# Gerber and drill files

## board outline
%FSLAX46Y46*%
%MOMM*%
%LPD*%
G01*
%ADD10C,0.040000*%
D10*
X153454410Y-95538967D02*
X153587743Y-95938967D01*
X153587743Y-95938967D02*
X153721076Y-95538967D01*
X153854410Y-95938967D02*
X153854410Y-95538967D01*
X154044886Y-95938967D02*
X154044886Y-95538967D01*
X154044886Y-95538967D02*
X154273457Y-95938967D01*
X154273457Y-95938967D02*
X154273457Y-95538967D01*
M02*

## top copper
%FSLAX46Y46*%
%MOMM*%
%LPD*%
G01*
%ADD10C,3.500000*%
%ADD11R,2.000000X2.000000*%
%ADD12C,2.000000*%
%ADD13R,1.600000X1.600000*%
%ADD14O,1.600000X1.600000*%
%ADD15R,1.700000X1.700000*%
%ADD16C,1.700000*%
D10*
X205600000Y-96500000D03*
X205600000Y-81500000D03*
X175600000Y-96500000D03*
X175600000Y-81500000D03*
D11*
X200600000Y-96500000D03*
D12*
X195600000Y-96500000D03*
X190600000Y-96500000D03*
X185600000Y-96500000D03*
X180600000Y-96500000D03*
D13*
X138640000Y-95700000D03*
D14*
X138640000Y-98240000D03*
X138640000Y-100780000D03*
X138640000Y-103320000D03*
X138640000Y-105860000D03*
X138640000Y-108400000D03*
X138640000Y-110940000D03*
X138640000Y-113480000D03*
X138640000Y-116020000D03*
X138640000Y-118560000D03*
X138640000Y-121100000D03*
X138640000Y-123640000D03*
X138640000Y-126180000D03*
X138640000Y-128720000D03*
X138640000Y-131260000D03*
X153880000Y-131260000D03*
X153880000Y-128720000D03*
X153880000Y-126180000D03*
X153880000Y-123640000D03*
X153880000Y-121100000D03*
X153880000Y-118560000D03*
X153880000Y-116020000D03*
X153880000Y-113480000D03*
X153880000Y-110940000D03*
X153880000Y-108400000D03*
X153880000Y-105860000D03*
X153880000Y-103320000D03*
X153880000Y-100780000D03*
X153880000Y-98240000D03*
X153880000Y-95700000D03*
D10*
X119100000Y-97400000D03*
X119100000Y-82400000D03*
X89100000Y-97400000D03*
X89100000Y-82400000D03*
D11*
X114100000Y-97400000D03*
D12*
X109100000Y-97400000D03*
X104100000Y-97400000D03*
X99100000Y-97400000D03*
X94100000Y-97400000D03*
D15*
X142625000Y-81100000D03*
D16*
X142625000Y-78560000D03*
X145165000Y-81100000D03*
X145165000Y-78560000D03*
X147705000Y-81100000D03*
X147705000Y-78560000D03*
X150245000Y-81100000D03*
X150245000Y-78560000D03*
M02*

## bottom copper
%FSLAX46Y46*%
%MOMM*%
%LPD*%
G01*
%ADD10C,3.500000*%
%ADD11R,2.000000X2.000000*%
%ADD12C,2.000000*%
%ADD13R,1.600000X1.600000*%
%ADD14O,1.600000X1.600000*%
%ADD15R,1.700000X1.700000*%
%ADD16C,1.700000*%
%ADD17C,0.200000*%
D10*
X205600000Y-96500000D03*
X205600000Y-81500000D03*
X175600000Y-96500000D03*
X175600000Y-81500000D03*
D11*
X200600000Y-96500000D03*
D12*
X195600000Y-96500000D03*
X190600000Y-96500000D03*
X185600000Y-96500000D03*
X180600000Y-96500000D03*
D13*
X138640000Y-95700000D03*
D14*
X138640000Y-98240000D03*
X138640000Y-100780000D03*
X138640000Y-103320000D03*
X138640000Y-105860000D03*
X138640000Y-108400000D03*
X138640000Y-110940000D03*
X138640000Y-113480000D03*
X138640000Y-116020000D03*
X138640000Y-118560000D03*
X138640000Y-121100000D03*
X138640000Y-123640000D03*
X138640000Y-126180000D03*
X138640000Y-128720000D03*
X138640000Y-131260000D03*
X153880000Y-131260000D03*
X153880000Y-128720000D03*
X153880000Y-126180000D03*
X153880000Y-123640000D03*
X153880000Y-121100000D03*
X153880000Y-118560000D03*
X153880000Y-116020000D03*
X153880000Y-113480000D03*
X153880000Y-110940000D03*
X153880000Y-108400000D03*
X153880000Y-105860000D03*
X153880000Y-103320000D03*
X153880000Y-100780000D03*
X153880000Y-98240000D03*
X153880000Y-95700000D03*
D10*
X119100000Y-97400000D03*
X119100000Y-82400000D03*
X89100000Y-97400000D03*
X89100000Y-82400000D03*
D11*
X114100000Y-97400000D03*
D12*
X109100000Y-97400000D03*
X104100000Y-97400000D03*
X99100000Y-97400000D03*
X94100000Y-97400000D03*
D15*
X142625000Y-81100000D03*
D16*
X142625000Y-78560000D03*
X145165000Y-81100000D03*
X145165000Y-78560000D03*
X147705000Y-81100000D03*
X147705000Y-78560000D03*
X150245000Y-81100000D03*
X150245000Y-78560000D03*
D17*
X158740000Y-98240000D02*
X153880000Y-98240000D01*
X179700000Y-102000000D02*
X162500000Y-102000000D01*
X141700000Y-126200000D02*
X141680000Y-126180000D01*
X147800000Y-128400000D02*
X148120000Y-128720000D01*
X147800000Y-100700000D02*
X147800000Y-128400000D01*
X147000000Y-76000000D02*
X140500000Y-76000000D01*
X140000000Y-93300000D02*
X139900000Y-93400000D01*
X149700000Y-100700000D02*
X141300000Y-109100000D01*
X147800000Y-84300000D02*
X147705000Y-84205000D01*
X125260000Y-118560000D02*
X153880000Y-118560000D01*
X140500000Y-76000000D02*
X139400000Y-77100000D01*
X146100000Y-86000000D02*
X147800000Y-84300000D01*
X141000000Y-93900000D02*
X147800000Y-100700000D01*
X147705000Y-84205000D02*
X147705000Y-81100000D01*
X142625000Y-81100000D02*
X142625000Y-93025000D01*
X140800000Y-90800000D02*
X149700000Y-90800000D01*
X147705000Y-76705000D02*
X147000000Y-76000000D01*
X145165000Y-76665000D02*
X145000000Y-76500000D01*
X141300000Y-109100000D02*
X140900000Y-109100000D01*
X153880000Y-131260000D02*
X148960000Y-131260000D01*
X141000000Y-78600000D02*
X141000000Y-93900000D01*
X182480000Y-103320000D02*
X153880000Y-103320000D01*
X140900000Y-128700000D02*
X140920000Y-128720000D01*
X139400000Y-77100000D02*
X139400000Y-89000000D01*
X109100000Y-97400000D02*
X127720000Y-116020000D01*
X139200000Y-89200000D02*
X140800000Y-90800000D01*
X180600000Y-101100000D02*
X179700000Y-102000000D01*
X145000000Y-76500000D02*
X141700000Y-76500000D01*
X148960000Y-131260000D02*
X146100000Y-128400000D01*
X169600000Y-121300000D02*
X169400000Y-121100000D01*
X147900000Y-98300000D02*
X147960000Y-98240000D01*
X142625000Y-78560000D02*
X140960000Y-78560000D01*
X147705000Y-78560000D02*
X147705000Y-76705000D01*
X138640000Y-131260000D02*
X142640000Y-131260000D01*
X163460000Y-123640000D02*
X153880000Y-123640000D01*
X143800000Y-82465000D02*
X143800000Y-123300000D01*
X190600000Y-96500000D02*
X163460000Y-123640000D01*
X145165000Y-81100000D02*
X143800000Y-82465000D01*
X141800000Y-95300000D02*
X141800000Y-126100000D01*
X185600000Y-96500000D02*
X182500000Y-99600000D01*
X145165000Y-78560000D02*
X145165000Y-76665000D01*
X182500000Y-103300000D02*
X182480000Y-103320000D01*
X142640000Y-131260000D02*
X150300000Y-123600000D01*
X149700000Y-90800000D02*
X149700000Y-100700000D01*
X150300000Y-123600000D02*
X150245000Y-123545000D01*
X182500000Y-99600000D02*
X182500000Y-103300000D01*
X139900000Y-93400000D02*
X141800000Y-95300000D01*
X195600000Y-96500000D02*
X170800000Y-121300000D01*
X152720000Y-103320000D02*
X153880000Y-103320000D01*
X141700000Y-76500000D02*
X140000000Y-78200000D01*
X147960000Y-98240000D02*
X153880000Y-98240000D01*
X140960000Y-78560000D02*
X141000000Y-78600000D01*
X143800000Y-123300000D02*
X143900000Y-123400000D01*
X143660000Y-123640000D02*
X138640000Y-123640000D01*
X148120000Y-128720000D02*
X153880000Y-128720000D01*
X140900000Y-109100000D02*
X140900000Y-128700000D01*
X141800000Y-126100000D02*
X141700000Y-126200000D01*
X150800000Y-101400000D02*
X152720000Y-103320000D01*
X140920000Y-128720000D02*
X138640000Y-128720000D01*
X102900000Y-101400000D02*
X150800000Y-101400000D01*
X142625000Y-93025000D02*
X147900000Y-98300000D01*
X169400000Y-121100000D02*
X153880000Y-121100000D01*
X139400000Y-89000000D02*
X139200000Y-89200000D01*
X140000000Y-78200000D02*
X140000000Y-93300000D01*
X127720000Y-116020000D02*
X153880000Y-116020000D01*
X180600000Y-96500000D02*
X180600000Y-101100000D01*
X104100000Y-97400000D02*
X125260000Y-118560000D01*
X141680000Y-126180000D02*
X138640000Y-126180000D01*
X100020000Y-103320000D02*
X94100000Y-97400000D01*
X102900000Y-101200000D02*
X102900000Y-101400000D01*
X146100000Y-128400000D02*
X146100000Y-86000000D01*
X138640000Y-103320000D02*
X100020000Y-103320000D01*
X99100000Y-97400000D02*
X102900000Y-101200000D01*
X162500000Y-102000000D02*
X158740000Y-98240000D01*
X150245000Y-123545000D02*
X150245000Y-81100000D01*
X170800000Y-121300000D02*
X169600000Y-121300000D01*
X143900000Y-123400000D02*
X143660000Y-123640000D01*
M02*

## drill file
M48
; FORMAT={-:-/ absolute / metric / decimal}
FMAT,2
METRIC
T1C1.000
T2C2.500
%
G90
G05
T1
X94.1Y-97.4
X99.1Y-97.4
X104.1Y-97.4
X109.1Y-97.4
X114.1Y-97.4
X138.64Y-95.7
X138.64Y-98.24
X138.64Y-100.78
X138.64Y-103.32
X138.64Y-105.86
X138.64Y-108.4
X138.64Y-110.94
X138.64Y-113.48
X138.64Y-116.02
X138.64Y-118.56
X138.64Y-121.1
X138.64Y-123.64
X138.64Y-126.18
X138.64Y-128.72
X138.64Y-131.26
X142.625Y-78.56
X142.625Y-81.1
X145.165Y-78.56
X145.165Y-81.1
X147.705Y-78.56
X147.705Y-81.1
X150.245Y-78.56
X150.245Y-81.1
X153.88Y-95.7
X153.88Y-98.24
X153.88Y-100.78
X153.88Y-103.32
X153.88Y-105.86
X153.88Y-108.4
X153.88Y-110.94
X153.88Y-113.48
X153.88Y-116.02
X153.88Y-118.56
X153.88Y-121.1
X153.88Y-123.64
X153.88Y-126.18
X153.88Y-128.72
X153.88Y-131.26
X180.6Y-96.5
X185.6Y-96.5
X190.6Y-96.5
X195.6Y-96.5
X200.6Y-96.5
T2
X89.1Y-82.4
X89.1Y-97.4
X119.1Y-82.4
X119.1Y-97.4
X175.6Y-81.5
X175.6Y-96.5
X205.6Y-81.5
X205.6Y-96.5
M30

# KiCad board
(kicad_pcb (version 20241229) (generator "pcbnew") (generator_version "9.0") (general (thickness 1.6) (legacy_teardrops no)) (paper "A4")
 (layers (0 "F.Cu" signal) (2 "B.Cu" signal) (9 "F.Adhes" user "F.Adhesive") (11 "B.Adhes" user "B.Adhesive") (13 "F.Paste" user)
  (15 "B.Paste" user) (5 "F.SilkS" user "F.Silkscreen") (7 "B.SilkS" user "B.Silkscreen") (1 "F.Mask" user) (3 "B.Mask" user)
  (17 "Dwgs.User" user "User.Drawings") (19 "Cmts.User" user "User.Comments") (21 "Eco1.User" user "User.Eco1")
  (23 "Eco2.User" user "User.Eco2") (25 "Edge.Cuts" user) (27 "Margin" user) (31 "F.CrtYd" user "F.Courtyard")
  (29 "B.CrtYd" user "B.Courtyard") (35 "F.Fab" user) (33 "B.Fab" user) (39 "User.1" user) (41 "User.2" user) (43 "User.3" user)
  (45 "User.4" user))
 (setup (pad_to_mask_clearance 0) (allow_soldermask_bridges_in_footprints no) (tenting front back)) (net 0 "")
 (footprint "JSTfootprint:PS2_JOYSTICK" (layer "F.Cu") (at 190.6 89 180)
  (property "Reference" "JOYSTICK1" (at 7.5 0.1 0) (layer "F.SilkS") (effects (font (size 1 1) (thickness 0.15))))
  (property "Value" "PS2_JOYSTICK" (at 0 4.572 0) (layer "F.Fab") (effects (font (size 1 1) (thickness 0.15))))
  (pad "" thru_hole circle (at -15 -7.5 180) (size 3.5 3.5) (drill 2.5) (layers "*.Cu" "*.Mask") (remove_unused_layers no))
  (pad "" thru_hole circle (at -15 7.5 180) (size 3.5 3.5) (drill 2.5) (layers "*.Cu" "*.Mask") (remove_unused_layers no))
  (pad "" thru_hole circle (at 15 -7.5 180) (size 3.5 3.5) (drill 2.5) (layers "*.Cu" "*.Mask") (remove_unused_layers no))
  (pad "" thru_hole circle (at 15 7.5 180) (size 3.5 3.5) (drill 2.5) (layers "*.Cu" "*.Mask") (remove_unused_layers no))
  (pad "1" thru_hole rect (at -10 -7.5 180) (size 2 2) (drill 1) (layers "*.Cu" "*.Mask") (remove_unused_layers no))
  (pad "2" thru_hole circle (at -5 -7.5 180) (size 2 2) (drill 1) (layers "*.Cu" "*.Mask") (remove_unused_layers no))
  (pad "3" thru_hole circle (at 0 -7.5 180) (size 2 2) (drill 1) (layers "*.Cu" "*.Mask") (remove_unused_layers no))
  (pad "4" thru_hole circle (at 5 -7.5 180) (size 2 2) (drill 1) (layers "*.Cu" "*.Mask") (remove_unused_layers no))
  (pad "5" thru_hole circle (at 10 -7.5 180) (size 2 2) (drill 1) (layers "*.Cu" "*.Mask") (remove_unused_layers no)))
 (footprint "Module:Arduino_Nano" (layer "F.Cu") (at 138.64 95.7)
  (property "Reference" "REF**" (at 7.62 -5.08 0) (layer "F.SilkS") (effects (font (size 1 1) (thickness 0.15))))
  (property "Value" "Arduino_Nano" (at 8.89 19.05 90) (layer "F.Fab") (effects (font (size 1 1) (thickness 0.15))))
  (pad "1" thru_hole rect (at 0 0) (size 1.6 1.6) (drill 1) (layers "*.Cu" "*.Mask") (remove_unused_layers no))
  (pad "2" thru_hole oval (at 0 2.54) (size 1.6 1.6) (drill 1) (layers "*.Cu" "*.Mask") (remove_unused_layers no))
  (pad "3" thru_hole oval (at 0 5.08) (size 1.6 1.6) (drill 1) (layers "*.Cu" "*.Mask") (remove_unused_layers no))
  (pad "4" thru_hole oval (at 0 7.62) (size 1.6 1.6) (drill 1) (layers "*.Cu" "*.Mask") (remove_unused_layers no))
  (pad "5" thru_hole oval (at 0 10.16) (size 1.6 1.6) (drill 1) (layers "*.Cu" "*.Mask") (remove_unused_layers no))
  (pad "6" thru_hole oval (at 0 12.7) (size 1.6 1.6) (drill 1) (layers "*.Cu" "*.Mask") (remove_unused_layers no))
  (pad "7" thru_hole oval (at 0 15.24) (size 1.6 1.6) (drill 1) (layers "*.Cu" "*.Mask") (remove_unused_layers no))
  (pad "8" thru_hole oval (at 0 17.78) (size 1.6 1.6) (drill 1) (layers "*.Cu" "*.Mask") (remove_unused_layers no))
  (pad "9" thru_hole oval (at 0 20.32) (size 1.6 1.6) (drill 1) (layers "*.Cu" "*.Mask") (remove_unused_layers no))
  (pad "10" thru_hole oval (at 0 22.86) (size 1.6 1.6) (drill 1) (layers "*.Cu" "*.Mask") (remove_unused_layers no))
  (pad "11" thru_hole oval (at 0 25.4) (size 1.6 1.6) (drill 1) (layers "*.Cu" "*.Mask") (remove_unused_layers no))
  (pad "12" thru_hole oval (at 0 27.94) (size 1.6 1.6) (drill 1) (layers "*.Cu" "*.Mask") (remove_unused_layers no))
  (pad "13" thru_hole oval (at 0 30.48) (size 1.6 1.6) (drill 1) (layers "*.Cu" "*.Mask") (remove_unused_layers no))
  (pad "14" thru_hole oval (at 0 33.02) (size 1.6 1.6) (drill 1) (layers "*.Cu" "*.Mask") (remove_unused_layers no))
  (pad "15" thru_hole oval (at 0 35.56) (size 1.6 1.6) (drill 1) (layers "*.Cu" "*.Mask") (remove_unused_layers no))
  (pad "16" thru_hole oval (at 15.24 35.56) (size 1.6 1.6) (drill 1) (layers "*.Cu" "*.Mask") (remove_unused_layers no))
  (pad "17" thru_hole oval (at 15.24 33.02) (size 1.6 1.6) (drill 1) (layers "*.Cu" "*.Mask") (remove_unused_layers no))
  (pad "18" thru_hole oval (at 15.24 30.48) (size 1.6 1.6) (drill 1) (layers "*.Cu" "*.Mask") (remove_unused_layers no))
  (pad "19" thru_hole oval (at 15.24 27.94) (size 1.6 1.6) (drill 1) (layers "*.Cu" "*.Mask") (remove_unused_layers no))
  (pad "20" thru_hole oval (at 15.24 25.4) (size 1.6 1.6) (drill 1) (layers "*.Cu" "*.Mask") (remove_unused_layers no))
  (pad "21" thru_hole oval (at 15.24 22.86) (size 1.6 1.6) (drill 1) (layers "*.Cu" "*.Mask") (remove_unused_layers no))
  (pad "22" thru_hole oval (at 15.24 20.32) (size 1.6 1.6) (drill 1) (layers "*.Cu" "*.Mask") (remove_unused_layers no))
  (pad "23" thru_hole oval (at 15.24 17.78) (size 1.6 1.6) (drill 1) (layers "*.Cu" "*.Mask") (remove_unused_layers no))
  (pad "24" thru_hole oval (at 15.24 15.24) (size 1.6 1.6) (drill 1) (layers "*.Cu" "*.Mask") (remove_unused_layers no))
  (pad "25" thru_hole oval (at 15.24 12.7) (size 1.6 1.6) (drill 1) (layers "*.Cu" "*.Mask") (remove_unused_layers no))
  (pad "26" thru_hole oval (at 15.24 10.16) (size 1.6 1.6) (drill 1) (layers "*.Cu" "*.Mask") (remove_unused_layers no))
  (pad "27" thru_hole oval (at 15.24 7.62) (size 1.6 1.6) (drill 1) (layers "*.Cu" "*.Mask") (remove_unused_layers no))
  (pad "28" thru_hole oval (at 15.24 5.08) (size 1.6 1.6) (drill 1) (layers "*.Cu" "*.Mask") (remove_unused_layers no))
  (pad "29" thru_hole oval (at 15.24 2.54) (size 1.6 1.6) (drill 1) (layers "*.Cu" "*.Mask") (remove_unused_layers no))
  (pad "30" thru_hole oval (at 15.24 0) (size 1.6 1.6) (drill 1) (layers "*.Cu" "*.Mask") (remove_unused_layers no)))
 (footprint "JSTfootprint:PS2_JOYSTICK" (layer "F.Cu") (at 104.1 89.9 180)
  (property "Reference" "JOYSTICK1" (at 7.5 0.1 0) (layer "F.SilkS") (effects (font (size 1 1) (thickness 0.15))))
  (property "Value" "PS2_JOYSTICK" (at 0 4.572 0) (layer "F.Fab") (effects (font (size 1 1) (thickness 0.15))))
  (pad "" thru_hole circle (at -15 -7.5 180) (size 3.5 3.5) (drill 2.5) (layers "*.Cu" "*.Mask") (remove_unused_layers no))
  (pad "" thru_hole circle (at -15 7.5 180) (size 3.5 3.5) (drill 2.5) (layers "*.Cu" "*.Mask") (remove_unused_layers no))
  (pad "" thru_hole circle (at 15 -7.5 180) (size 3.5 3.5) (drill 2.5) (layers "*.Cu" "*.Mask") (remove_unused_layers no))
  (pad "" thru_hole circle (at 15 7.5 180) (size 3.5 3.5) (drill 2.5) (layers "*.Cu" "*.Mask") (remove_unused_layers no))
  (pad "1" thru_hole rect (at -10 -7.5 180) (size 2 2) (drill 1) (layers "*.Cu" "*.Mask") (remove_unused_layers no))
  (pad "2" thru_hole circle (at -5 -7.5 180) (size 2 2) (drill 1) (layers "*.Cu" "*.Mask") (remove_unused_layers no))
  (pad "3" thru_hole circle (at 0 -7.5 180) (size 2 2) (drill 1) (layers "*.Cu" "*.Mask") (remove_unused_layers no))
  (pad "4" thru_hole circle (at 5 -7.5 180) (size 2 2) (drill 1) (layers "*.Cu" "*.Mask") (remove_unused_layers no))
  (pad "5" thru_hole circle (at 10 -7.5 180) (size 2 2) (drill 1) (layers "*.Cu" "*.Mask") (remove_unused_layers no)))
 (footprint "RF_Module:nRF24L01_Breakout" (layer "F.Cu") (at 142.625 81.1 90)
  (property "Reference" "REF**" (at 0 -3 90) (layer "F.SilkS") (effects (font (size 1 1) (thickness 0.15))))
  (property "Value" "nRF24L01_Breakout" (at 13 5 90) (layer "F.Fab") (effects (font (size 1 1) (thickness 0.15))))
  (pad "1" thru_hole rect (at 0 0 90) (size 1.7 1.7) (drill 1) (layers "*.Cu" "*.Mask") (remove_unused_layers no))
  (pad "2" thru_hole circle (at 2.54 0 90) (size 1.7 1.7) (drill 1) (layers "*.Cu" "*.Mask") (remove_unused_layers no))
  (pad "3" thru_hole circle (at 0 2.54 90) (size 1.7 1.7) (drill 1) (layers "*.Cu" "*.Mask") (remove_unused_layers no))
  (pad "4" thru_hole circle (at 2.54 2.54 90) (size 1.7 1.7) (drill 1) (layers "*.Cu" "*.Mask") (remove_unused_layers no))
  (pad "5" thru_hole circle (at 0 5.08 90) (size 1.7 1.7) (drill 1) (layers "*.Cu" "*.Mask") (remove_unused_layers no))
  (pad "6" thru_hole circle (at 2.54 5.08 90) (size 1.7 1.7) (drill 1) (layers "*.Cu" "*.Mask") (remove_unused_layers no))
  (pad "7" thru_hole circle (at 0 7.62 90) (size 1.7 1.7) (drill 1) (layers "*.Cu" "*.Mask") (remove_unused_layers no))
  (pad "8" thru_hole circle (at 2.54 7.62 90) (size 1.7 1.7) (drill 1) (layers "*.Cu" "*.Mask") (remove_unused_layers no)))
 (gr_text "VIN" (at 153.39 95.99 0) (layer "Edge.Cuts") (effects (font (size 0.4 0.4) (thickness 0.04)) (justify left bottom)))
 (segment (start 158.74 98.24) (end 153.88 98.24) (width 0.2) (layer "B.Cu") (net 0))
 (segment (start 179.7 102) (end 162.5 102) (width 0.2) (layer "B.Cu") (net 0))
 (segment (start 141.7 126.2) (end 141.68 126.18) (width 0.2) (layer "B.Cu") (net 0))
 (segment (start 147.8 128.4) (end 148.12 128.72) (width 0.2) (layer "B.Cu") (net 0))
 (segment (start 147.8 100.7) (end 147.8 128.4) (width 0.2) (layer "B.Cu") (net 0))
 (segment (start 147 76) (end 140.5 76) (width 0.2) (layer "B.Cu") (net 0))
 (segment (start 140 93.3) (end 139.9 93.4) (width 0.2) (layer "B.Cu") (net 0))
 (segment (start 149.7 100.7) (end 141.3 109.1) (width 0.2) (layer "B.Cu") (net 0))
 (segment (start 147.8 84.3) (end 147.705 84.205) (width 0.2) (layer "B.Cu") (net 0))
 (segment (start 125.26 118.56) (end 153.88 118.56) (width 0.2) (layer "B.Cu") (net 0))
 (segment (start 140.5 76) (end 139.4 77.1) (width 0.2) (layer "B.Cu") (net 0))
 (segment (start 146.1 86) (end 147.8 84.3) (width 0.2) (layer "B.Cu") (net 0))
 (segment (start 141 93.9) (end 147.8 100.7) (width 0.2) (layer "B.Cu") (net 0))
 (segment (start 147.705 84.205) (end 147.705 81.1) (width 0.2) (layer "B.Cu") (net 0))
 (segment (start 142.625 81.1) (end 142.625 93.025) (width 0.2) (layer "B.Cu") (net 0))
 (segment (start 140.8 90.8) (end 149.7 90.8) (width 0.2) (layer "B.Cu") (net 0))
 (segment (start 147.705 76.705) (end 147 76) (width 0.2) (layer "B.Cu") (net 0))
 (segment (start 145.165 76.665) (end 145 76.5) (width 0.2) (layer "B.Cu") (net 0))
 (segment (start 141.3 109.1) (end 140.9 109.1) (width 0.2) (layer "B.Cu") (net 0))
 (segment (start 153.88 131.26) (end 148.96 131.26) (width 0.2) (layer "B.Cu") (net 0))
 (segment (start 141 78.6) (end 141 93.9) (width 0.2) (layer "B.Cu") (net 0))
 (segment (start 182.48 103.32) (end 153.88 103.32) (width 0.2) (layer "B.Cu") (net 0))
 (segment (start 140.9 128.7) (end 140.92 128.72) (width 0.2) (layer "B.Cu") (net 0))
 (segment (start 139.4 77.1) (end 139.4 89) (width 0.2) (layer "B.Cu") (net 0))
 (segment (start 109.1 97.4) (end 127.72 116.02) (width 0.2) (layer "B.Cu") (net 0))
 (segment (start 139.2 89.2) (end 140.8 90.8) (width 0.2) (layer "B.Cu") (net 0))
 (segment (start 180.6 101.1) (end 179.7 102) (width 0.2) (layer "B.Cu") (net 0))
 (segment (start 145 76.5) (end 141.7 76.5) (width 0.2) (layer "B.Cu") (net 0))
 (segment (start 148.96 131.26) (end 146.1 128.4) (width 0.2) (layer "B.Cu") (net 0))
 (segment (start 169.6 121.3) (end 169.4 121.1) (width 0.2) (layer "B.Cu") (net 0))
 (segment (start 147.9 98.3) (end 147.96 98.24) (width 0.2) (layer "B.Cu") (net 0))
 (segment (start 142.625 78.56) (end 140.96 78.56) (width 0.2) (layer "B.Cu") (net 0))
 (segment (start 147.705 78.56) (end 147.705 76.705) (width 0.2) (layer "B.Cu") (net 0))
 (segment (start 138.64 131.26) (end 142.64 131.26) (width 0.2) (layer "B.Cu") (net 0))
 (segment (start 163.46 123.64) (end 153.88 123.64) (width 0.2) (layer "B.Cu") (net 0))
 (segment (start 143.8 82.465) (end 143.8 123.3) (width 0.2) (layer "B.Cu") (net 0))
 (segment (start 190.6 96.5) (end 163.46 123.64) (width 0.2) (layer "B.Cu") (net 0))
 (segment (start 145.165 81.1) (end 143.8 82.465) (width 0.2) (layer "B.Cu") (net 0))
 (segment (start 141.8 95.3) (end 141.8 126.1) (width 0.2) (layer "B.Cu") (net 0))
 (segment (start 185.6 96.5) (end 182.5 99.6) (width 0.2) (layer "B.Cu") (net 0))
 (segment (start 145.165 78.56) (end 145.165 76.665) (width 0.2) (layer "B.Cu") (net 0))
 (segment (start 182.5 103.3) (end 182.48 103.32) (width 0.2) (layer "B.Cu") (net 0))
 (segment (start 142.64 131.26) (end 150.3 123.6) (width 0.2) (layer "B.Cu") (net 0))
 (segment (start 149.7 90.8) (end 149.7 100.7) (width 0.2) (layer "B.Cu") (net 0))
 (segment (start 150.3 123.6) (end 150.245 123.545) (width 0.2) (layer "B.Cu") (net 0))
 (segment (start 182.5 99.6) (end 182.5 103.3) (width 0.2) (layer "B.Cu") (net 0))
 (segment (start 139.9 93.4) (end 141.8 95.3) (width 0.2) (layer "B.Cu") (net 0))
 (segment (start 195.6 96.5) (end 170.8 121.3) (width 0.2) (layer "B.Cu") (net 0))
 (segment (start 152.72 103.32) (end 153.88 103.32) (width 0.2) (layer "B.Cu") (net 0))
 (segment (start 141.7 76.5) (end 140 78.2) (width 0.2) (layer "B.Cu") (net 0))
 (segment (start 147.96 98.24) (end 153.88 98.24) (width 0.2) (layer "B.Cu") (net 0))
 (segment (start 140.96 78.56) (end 141 78.6) (width 0.2) (layer "B.Cu") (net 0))
 (segment (start 143.8 123.3) (end 143.9 123.4) (width 0.2) (layer "B.Cu") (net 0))
 (segment (start 143.66 123.64) (end 138.64 123.64) (width 0.2) (layer "B.Cu") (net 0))
 (segment (start 148.12 128.72) (end 153.88 128.72) (width 0.2) (layer "B.Cu") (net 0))
 (segment (start 140.9 109.1) (end 140.9 128.7) (width 0.2) (layer "B.Cu") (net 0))
 (segment (start 141.8 126.1) (end 141.7 126.2) (width 0.2) (layer "B.Cu") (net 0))
 (segment (start 150.8 101.4) (end 152.72 103.32) (width 0.2) (layer "B.Cu") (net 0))
 (segment (start 140.92 128.72) (end 138.64 128.72) (width 0.2) (layer "B.Cu") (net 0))
 (segment (start 102.9 101.4) (end 150.8 101.4) (width 0.2) (layer "B.Cu") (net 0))
 (segment (start 142.625 93.025) (end 147.9 98.3) (width 0.2) (layer "B.Cu") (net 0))
 (segment (start 169.4 121.1) (end 153.88 121.1) (width 0.2) (layer "B.Cu") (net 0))
 (segment (start 139.4 89) (end 139.2 89.2) (width 0.2) (layer "B.Cu") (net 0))
 (segment (start 140 78.2) (end 140 93.3) (width 0.2) (layer "B.Cu") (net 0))
 (segment (start 127.72 116.02) (end 153.88 116.02) (width 0.2) (layer "B.Cu") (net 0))
 (segment (start 180.6 96.5) (end 180.6 101.1) (width 0.2) (layer "B.Cu") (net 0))
 (segment (start 104.1 97.4) (end 125.26 118.56) (width 0.2) (layer "B.Cu") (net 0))
 (segment (start 141.68 126.18) (end 138.64 126.18) (width 0.2) (layer "B.Cu") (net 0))
 (segment (start 100.02 103.32) (end 94.1 97.4) (width 0.2) (layer "B.Cu") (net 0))
 (segment (start 102.9 101.2) (end 102.9 101.4) (width 0.2) (layer "B.Cu") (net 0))
 (segment (start 146.1 128.4) (end 146.1 86) (width 0.2) (layer "B.Cu") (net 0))
 (segment (start 138.64 103.32) (end 100.02 103.32) (width 0.2) (layer "B.Cu") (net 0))
 (segment (start 99.1 97.4) (end 102.9 101.2) (width 0.2) (layer "B.Cu") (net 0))
 (segment (start 162.5 102) (end 158.74 98.24) (width 0.2) (layer "B.Cu") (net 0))
 (segment (start 150.245 123.545) (end 150.245 81.1) (width 0.2) (layer "B.Cu") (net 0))
 (segment (start 170.8 121.3) (end 169.6 121.3) (width 0.2) (layer "B.Cu") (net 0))
 (segment (start 143.9 123.4) (end 143.66 123.64) (width 0.2) (layer "B.Cu") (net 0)))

